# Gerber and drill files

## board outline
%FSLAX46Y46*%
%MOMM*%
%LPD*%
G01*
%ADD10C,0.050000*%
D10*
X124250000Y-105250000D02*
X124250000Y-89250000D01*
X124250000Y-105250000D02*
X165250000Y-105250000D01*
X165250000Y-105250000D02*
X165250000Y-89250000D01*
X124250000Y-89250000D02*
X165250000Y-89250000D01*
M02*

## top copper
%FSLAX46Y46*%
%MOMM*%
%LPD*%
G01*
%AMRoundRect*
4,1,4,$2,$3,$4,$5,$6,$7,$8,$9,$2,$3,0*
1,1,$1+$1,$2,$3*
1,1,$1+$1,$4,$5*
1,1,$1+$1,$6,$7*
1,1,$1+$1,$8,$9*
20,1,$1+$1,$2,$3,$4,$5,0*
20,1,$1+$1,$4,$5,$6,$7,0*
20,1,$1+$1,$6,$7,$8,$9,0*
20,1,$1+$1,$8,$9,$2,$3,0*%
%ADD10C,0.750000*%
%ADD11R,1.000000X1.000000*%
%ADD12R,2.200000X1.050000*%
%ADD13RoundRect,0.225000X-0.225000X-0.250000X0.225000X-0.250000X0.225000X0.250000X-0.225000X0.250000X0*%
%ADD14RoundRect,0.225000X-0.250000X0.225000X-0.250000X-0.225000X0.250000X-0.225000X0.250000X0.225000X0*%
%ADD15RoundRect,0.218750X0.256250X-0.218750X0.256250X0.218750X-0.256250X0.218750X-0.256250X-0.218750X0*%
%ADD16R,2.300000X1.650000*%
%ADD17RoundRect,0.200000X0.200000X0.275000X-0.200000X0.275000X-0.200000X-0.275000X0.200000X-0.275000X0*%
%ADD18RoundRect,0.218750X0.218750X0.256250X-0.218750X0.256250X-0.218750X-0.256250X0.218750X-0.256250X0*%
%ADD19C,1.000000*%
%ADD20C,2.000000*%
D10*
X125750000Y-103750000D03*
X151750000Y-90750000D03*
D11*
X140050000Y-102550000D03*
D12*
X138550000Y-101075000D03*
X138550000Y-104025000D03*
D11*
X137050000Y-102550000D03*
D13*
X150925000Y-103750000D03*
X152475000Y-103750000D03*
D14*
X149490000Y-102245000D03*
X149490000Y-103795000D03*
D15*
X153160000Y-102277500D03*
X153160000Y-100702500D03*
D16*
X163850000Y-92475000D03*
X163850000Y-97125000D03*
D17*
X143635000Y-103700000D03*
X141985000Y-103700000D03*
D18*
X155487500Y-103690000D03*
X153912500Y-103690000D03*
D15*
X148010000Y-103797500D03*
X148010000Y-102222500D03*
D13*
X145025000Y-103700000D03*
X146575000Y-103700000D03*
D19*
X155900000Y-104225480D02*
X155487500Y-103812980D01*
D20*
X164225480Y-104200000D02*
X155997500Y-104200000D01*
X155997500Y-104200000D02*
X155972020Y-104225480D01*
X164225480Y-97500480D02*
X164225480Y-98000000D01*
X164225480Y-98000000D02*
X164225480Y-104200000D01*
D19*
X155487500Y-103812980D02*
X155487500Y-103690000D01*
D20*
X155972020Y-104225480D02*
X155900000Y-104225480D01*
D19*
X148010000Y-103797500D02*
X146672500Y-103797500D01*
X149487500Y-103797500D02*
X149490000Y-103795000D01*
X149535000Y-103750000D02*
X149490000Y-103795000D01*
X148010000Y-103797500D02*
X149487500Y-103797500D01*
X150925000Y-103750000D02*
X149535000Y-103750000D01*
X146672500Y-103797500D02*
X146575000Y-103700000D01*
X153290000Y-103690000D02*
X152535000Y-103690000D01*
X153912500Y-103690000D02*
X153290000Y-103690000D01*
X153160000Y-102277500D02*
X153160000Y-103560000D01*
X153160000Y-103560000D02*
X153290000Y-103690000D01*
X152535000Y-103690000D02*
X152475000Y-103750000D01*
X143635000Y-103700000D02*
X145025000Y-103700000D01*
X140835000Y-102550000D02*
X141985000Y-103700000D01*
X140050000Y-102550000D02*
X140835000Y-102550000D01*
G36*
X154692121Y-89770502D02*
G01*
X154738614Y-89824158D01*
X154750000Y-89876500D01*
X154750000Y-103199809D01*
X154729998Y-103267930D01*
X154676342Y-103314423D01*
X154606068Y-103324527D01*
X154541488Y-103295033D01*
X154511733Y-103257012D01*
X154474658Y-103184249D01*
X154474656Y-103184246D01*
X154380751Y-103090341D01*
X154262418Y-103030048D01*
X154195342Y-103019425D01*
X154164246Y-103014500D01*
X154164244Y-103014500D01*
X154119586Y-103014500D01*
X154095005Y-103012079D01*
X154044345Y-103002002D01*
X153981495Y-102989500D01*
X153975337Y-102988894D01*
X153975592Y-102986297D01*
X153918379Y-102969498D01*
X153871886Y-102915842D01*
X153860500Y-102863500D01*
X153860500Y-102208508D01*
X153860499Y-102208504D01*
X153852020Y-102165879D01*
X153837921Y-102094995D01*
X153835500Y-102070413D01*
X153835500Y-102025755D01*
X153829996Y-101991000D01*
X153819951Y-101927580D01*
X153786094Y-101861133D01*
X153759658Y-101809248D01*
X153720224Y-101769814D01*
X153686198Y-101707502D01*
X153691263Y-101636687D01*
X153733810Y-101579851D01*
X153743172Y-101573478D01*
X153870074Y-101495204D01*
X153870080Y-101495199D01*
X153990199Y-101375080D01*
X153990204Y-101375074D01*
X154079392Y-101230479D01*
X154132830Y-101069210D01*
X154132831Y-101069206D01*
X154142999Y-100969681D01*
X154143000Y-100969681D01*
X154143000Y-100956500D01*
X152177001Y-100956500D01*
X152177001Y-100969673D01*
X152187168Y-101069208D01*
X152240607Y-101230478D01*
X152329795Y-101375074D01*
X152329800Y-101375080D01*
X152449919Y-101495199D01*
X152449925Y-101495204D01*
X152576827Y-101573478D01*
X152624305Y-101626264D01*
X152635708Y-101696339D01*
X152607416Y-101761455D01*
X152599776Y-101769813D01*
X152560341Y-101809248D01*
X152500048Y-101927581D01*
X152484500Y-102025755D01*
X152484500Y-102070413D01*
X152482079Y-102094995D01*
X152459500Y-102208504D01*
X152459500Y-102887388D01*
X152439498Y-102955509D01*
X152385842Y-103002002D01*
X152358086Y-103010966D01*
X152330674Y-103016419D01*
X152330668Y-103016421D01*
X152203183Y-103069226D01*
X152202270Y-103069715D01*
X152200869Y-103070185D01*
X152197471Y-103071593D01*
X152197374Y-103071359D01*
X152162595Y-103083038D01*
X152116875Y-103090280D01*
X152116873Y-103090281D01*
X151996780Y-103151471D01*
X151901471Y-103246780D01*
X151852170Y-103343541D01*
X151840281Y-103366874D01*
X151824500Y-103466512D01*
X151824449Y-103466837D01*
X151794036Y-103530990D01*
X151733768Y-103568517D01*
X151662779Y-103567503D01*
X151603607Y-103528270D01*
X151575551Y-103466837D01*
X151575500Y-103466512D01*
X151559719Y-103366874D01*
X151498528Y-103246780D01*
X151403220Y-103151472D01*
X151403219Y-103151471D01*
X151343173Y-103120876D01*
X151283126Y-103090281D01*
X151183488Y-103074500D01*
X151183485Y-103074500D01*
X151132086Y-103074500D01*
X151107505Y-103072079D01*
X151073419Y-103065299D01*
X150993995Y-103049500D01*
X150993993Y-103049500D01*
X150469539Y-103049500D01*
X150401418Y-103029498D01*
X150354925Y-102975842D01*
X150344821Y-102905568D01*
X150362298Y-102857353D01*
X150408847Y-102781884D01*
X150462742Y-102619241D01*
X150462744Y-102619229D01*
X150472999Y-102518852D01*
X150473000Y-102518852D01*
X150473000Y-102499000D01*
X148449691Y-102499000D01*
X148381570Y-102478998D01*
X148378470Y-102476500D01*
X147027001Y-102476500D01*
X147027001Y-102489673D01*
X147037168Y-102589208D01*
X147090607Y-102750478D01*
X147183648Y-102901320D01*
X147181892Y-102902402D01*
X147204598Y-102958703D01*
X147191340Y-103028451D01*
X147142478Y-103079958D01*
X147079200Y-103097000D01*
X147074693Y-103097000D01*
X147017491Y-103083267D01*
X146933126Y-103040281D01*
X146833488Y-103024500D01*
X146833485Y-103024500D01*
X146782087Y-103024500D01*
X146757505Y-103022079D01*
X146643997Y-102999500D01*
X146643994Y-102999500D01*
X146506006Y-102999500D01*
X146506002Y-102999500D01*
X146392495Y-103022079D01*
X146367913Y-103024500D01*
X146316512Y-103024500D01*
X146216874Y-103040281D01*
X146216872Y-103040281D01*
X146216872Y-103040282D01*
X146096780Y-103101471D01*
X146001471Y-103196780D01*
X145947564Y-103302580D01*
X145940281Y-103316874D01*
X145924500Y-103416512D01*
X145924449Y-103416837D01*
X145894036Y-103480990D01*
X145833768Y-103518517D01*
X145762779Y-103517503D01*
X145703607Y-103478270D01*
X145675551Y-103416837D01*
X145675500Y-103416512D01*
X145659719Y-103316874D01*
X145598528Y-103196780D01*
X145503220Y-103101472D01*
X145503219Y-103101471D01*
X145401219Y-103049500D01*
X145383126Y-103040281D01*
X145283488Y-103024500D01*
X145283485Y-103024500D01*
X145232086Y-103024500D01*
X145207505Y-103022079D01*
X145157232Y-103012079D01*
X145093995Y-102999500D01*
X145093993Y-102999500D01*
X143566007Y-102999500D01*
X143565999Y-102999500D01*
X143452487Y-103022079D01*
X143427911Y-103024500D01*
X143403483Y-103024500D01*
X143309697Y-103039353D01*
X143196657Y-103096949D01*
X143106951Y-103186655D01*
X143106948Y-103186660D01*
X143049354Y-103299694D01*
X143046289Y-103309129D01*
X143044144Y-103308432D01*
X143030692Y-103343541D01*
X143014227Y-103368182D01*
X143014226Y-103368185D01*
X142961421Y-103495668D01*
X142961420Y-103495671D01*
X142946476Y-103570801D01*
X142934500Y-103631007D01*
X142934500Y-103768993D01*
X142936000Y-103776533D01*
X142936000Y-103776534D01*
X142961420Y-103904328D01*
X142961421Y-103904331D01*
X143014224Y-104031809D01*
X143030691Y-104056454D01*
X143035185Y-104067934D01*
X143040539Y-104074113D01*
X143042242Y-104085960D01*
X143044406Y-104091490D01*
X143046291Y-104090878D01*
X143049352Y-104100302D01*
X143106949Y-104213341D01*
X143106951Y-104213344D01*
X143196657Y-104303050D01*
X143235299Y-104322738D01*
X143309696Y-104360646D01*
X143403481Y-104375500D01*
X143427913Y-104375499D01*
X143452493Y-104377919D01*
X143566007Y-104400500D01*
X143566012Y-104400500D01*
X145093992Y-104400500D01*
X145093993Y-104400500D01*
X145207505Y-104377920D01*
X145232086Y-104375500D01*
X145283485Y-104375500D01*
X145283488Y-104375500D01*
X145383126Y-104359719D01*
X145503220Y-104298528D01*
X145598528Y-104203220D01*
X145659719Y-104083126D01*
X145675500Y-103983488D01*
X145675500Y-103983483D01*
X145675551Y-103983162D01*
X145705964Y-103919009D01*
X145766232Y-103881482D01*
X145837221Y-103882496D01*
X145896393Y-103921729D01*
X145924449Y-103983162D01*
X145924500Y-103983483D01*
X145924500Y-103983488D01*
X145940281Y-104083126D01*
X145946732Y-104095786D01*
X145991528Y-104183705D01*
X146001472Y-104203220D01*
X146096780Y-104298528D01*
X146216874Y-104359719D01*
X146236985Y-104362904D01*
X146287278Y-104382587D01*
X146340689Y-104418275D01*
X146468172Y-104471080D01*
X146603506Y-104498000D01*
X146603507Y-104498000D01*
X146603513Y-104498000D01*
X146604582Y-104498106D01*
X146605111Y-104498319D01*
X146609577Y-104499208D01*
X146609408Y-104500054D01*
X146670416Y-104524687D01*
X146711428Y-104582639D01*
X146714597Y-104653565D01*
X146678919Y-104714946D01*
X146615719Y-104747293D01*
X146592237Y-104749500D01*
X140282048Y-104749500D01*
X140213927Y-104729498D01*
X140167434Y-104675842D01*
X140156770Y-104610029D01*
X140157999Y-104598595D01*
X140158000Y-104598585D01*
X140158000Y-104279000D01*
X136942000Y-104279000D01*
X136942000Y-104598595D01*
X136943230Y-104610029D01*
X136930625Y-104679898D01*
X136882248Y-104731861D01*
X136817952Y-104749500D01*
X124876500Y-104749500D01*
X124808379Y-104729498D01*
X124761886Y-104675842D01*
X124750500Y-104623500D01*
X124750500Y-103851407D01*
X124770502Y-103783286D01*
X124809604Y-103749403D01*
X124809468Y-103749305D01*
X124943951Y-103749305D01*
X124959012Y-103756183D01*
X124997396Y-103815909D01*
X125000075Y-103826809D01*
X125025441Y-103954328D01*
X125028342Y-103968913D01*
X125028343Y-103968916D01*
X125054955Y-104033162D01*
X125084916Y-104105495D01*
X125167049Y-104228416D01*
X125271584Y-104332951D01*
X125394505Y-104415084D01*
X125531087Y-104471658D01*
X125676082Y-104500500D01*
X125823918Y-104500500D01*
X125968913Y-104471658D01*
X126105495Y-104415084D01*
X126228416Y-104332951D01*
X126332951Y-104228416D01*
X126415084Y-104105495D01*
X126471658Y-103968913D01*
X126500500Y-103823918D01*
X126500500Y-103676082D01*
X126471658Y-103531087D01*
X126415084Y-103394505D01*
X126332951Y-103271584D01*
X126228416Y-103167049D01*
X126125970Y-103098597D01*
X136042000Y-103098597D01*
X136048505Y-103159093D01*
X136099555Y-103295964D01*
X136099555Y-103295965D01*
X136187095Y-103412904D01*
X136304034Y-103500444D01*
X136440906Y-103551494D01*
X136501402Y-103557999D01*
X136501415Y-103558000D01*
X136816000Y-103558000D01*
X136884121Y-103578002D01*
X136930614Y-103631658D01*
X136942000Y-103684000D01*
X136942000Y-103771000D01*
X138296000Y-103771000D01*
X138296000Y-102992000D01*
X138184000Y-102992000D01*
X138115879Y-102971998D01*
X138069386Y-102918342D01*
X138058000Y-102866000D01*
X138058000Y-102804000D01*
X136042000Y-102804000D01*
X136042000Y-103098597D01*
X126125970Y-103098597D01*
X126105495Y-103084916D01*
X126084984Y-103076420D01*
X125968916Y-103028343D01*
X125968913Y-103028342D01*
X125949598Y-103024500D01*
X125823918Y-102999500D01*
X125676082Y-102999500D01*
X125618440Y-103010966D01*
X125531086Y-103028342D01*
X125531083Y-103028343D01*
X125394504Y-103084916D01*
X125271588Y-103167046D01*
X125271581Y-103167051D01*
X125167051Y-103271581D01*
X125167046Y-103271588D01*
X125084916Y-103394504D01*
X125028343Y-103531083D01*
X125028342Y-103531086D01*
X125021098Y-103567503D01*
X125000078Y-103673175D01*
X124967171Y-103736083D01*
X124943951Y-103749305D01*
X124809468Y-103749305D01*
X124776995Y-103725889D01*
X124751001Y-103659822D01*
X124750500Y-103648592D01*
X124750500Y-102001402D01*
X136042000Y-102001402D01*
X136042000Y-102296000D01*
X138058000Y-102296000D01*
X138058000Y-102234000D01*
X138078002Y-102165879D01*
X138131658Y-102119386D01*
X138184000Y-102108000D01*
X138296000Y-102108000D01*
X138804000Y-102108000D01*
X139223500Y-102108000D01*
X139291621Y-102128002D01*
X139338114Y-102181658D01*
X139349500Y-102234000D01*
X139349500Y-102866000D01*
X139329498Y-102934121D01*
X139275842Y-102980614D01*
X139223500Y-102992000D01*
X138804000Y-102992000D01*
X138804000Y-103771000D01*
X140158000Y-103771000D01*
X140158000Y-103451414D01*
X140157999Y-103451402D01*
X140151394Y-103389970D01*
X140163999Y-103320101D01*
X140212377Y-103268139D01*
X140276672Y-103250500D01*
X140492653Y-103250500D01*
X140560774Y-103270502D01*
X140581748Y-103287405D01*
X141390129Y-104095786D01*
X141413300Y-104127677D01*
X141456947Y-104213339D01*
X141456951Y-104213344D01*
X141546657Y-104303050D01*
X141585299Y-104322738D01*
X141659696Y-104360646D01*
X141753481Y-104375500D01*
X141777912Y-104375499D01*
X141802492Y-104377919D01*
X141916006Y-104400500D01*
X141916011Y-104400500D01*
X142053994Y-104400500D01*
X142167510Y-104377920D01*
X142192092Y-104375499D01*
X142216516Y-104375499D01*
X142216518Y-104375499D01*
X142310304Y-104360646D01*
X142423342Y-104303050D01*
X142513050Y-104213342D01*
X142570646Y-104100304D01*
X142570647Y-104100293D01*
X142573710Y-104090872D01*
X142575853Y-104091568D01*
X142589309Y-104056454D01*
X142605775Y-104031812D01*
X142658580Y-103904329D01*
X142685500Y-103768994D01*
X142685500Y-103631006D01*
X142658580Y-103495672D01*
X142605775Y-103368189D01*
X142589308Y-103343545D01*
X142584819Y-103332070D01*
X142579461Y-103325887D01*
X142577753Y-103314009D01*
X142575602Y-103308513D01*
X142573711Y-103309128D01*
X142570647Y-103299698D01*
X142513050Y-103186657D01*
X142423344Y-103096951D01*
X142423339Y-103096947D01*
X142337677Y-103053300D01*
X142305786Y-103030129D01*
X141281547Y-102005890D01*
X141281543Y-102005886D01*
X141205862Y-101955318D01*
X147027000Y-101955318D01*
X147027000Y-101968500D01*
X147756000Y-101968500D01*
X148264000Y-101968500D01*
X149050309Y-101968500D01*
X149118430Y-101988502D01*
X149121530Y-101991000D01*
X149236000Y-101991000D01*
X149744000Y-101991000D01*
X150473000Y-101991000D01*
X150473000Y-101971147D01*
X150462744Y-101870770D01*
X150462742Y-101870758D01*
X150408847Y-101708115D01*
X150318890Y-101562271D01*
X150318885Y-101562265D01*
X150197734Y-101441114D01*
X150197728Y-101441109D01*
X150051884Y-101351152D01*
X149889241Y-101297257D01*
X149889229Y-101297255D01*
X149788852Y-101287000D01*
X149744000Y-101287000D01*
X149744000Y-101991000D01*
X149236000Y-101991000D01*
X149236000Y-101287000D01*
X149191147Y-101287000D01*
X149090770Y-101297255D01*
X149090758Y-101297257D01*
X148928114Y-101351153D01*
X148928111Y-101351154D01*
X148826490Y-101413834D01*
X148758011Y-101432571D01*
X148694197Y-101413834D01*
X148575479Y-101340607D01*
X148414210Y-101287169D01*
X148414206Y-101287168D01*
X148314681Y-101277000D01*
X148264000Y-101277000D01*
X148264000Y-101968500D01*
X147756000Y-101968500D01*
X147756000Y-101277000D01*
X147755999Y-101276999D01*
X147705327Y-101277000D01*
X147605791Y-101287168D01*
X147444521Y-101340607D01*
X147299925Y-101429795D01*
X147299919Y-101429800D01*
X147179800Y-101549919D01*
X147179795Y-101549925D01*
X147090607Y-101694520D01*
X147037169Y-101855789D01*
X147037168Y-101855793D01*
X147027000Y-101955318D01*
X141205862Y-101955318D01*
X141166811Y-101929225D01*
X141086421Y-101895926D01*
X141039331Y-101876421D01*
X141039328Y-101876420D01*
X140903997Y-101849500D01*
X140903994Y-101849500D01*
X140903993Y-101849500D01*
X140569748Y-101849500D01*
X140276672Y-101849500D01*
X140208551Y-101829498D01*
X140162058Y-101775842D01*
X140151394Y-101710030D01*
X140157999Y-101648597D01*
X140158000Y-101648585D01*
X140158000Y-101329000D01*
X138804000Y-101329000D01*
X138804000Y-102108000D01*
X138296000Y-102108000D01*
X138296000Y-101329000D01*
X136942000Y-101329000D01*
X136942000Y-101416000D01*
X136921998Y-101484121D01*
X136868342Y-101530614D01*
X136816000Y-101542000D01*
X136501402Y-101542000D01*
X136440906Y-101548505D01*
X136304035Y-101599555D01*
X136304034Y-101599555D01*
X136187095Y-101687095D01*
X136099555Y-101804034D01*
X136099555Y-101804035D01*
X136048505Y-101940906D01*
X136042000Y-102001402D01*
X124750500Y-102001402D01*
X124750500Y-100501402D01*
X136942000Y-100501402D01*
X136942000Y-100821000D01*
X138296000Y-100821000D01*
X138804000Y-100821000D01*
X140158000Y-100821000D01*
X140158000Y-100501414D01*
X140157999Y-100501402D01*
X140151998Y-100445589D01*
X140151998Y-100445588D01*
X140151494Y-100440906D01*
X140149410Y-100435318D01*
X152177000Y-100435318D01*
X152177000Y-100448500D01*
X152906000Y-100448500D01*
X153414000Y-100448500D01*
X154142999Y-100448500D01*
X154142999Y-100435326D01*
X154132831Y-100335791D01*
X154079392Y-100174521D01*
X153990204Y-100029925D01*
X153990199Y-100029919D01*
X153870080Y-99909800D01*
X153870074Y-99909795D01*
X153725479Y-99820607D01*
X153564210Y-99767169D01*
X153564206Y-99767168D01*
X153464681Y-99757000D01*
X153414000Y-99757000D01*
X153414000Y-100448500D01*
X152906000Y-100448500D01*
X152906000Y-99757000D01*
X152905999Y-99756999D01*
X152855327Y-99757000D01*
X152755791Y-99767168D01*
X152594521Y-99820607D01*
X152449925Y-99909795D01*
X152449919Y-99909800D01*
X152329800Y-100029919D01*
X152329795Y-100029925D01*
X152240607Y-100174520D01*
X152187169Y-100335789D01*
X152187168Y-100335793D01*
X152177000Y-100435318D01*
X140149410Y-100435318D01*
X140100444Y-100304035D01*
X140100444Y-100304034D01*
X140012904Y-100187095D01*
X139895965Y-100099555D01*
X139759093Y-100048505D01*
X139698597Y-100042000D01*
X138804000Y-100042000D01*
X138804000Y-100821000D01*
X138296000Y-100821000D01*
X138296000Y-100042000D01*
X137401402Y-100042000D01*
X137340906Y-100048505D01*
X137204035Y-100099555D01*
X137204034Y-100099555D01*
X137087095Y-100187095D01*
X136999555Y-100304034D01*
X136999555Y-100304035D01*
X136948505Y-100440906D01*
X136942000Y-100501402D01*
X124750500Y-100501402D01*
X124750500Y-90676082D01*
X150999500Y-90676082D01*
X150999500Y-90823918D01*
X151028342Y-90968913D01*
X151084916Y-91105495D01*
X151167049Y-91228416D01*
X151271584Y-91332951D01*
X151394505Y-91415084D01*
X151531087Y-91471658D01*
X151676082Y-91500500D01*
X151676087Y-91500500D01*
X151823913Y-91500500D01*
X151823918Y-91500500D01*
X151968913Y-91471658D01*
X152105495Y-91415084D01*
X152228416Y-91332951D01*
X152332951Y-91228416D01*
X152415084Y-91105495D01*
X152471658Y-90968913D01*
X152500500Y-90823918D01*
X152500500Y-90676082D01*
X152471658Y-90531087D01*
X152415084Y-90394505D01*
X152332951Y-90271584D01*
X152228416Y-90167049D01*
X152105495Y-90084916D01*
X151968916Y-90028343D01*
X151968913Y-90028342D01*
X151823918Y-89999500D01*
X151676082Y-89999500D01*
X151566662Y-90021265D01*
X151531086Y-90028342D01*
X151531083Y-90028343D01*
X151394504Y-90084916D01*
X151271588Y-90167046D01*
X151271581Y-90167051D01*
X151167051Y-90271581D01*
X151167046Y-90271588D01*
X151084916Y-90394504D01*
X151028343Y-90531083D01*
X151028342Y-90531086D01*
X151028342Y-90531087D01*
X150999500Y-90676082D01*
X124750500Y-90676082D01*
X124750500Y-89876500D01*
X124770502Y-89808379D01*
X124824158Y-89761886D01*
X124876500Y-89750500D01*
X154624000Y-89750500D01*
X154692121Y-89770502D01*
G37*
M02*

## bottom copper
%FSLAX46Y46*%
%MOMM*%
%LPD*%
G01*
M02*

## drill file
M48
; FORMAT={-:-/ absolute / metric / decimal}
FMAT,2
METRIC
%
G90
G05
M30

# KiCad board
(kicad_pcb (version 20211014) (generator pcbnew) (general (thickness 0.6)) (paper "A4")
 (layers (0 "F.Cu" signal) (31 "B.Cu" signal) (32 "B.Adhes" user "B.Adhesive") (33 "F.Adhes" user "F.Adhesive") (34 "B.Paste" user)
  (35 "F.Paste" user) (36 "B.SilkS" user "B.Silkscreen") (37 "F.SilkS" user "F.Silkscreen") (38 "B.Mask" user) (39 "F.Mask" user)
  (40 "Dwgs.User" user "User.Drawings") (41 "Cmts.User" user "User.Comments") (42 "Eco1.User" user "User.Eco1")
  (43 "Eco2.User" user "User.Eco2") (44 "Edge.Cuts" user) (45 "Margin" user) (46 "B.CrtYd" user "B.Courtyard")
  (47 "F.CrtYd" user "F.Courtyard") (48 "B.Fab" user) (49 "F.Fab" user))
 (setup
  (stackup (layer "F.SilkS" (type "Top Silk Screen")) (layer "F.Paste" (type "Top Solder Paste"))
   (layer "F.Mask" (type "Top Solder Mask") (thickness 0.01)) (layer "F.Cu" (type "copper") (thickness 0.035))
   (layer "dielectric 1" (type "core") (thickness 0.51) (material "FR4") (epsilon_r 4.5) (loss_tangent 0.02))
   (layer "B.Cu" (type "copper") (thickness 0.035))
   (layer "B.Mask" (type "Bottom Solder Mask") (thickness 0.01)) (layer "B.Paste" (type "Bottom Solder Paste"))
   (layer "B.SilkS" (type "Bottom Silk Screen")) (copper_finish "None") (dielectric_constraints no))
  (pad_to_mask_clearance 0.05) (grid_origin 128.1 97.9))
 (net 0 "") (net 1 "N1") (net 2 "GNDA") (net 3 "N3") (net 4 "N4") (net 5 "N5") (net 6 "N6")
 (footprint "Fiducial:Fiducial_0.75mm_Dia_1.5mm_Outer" (layer "F.Cu") (at 125.75 103.75)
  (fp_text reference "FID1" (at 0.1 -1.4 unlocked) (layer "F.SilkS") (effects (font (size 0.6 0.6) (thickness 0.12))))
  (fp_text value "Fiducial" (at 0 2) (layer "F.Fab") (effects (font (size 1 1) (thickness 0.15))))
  (pad "" smd circle locked (at 0 0) (size 0.75 0.75) (layers "F.Cu" "F.Mask") (solder_mask_margin 0.375) (clearance 0.375)))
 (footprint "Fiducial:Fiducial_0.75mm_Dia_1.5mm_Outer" (layer "F.Cu") (at 151.75 90.75)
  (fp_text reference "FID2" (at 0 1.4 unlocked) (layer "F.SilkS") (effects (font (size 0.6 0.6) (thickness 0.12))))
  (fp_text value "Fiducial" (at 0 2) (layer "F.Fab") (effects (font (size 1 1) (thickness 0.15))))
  (pad "" smd circle locked (at 0 0) (size 0.75 0.75) (layers "F.Cu" "F.Mask") (solder_mask_margin 0.375) (clearance 0.375)))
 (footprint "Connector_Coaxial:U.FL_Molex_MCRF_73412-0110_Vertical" (layer "F.Cu") (at 138.55 102.55 90)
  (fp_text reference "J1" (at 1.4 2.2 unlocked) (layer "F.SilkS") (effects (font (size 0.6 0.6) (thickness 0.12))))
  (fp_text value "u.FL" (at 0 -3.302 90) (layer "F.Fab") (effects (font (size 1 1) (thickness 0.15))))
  (pad "1" smd rect locked (at 0 1.5 90) (size 1 1) (layers "F.Cu" "F.Paste" "F.Mask") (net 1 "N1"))
  (pad "2" smd rect locked (at 1.475 0 90) (size 1.05 2.2) (layers "F.Cu" "F.Paste" "F.Mask") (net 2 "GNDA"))
  (pad "2" smd rect locked (at -1.475 0 90) (size 1.05 2.2) (layers "F.Cu" "F.Paste" "F.Mask") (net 2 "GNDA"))
  (pad "2" smd rect locked (at 0 -1.5 90) (size 1 1) (layers "F.Cu" "F.Paste" "F.Mask") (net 2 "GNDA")))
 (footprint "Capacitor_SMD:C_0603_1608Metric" (layer "F.Cu") (at 151.7 103.75)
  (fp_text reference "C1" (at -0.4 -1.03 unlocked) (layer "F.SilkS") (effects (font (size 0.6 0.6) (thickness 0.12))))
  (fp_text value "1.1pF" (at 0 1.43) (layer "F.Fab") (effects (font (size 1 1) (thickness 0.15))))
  (pad "1" smd roundrect locked (at -0.775 0) (size 0.9 0.95) (layers "F.Cu" "F.Paste" "F.Mask") (roundrect_rratio 0.25) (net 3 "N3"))
  (pad "2" smd roundrect locked (at 0.775 0) (size 0.9 0.95) (layers "F.Cu" "F.Paste" "F.Mask") (roundrect_rratio 0.25) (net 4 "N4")))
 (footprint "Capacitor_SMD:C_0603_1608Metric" (layer "F.Cu") (at 149.49 103.02 -90)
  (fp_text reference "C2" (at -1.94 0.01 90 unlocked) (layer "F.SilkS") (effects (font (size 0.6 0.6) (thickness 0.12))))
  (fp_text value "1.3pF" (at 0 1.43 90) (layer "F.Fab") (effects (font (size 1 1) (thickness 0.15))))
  (pad "1" smd roundrect locked (at -0.775 0 270) (size 0.9 0.95) (layers "F.Cu" "F.Paste" "F.Mask") (roundrect_rratio 0.25) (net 2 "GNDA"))
  (pad "2" smd roundrect locked (at 0.775 0 270) (size 0.9 0.95) (layers "F.Cu" "F.Paste" "F.Mask") (roundrect_rratio 0.25) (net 3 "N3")))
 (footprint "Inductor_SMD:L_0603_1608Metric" (layer "F.Cu") (at 153.16 101.49 90)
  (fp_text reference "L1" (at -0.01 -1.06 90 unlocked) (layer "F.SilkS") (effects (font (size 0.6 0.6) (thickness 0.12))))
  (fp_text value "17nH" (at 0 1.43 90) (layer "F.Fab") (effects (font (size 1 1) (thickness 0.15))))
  (pad "1" smd roundrect locked (at -0.7875 0 90) (size 0.875 0.95) (layers "F.Cu" "F.Paste" "F.Mask") (roundrect_rratio 0.25) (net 4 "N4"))
  (pad "2" smd roundrect locked (at 0.7875 0 90) (size 0.875 0.95) (layers "F.Cu" "F.Paste" "F.Mask") (roundrect_rratio 0.25) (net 2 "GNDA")))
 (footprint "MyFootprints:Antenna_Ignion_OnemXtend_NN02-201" (layer "F.Cu") (at 163.85 94.8 -90)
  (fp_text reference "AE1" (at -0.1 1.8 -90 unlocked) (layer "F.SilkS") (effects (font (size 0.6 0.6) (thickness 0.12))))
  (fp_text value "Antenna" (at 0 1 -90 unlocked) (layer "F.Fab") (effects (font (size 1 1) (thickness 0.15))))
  (pad "" smd rect (at -2.325 0 270) (size 1.65 2.3) (layers "F.Cu" "F.Paste" "F.Mask"))
  (pad "1" smd rect (at 2.325 0 270) (size 1.65 2.3) (layers "F.Cu" "F.Paste" "F.Mask") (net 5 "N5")))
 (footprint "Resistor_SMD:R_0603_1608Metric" (layer "F.Cu") (at 142.81 103.7 180)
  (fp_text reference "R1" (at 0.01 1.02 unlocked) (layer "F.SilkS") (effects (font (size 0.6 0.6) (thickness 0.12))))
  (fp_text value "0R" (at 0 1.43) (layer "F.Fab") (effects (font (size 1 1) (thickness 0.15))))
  (pad "1" smd roundrect locked (at -0.825 0 180) (size 0.8 0.95) (layers "F.Cu" "F.Paste" "F.Mask") (roundrect_rratio 0.25) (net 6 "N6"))
  (pad "2" smd roundrect locked (at 0.825 0 180) (size 0.8 0.95) (layers "F.Cu" "F.Paste" "F.Mask") (roundrect_rratio 0.25) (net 1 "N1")))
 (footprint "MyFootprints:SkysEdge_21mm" (layer "F.Cu") (at 133.3 91.8)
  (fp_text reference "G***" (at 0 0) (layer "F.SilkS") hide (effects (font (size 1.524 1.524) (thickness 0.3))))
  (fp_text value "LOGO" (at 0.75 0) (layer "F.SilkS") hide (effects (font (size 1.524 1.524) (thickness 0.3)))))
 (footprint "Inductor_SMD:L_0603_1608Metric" (layer "F.Cu") (at 154.7 103.69 180)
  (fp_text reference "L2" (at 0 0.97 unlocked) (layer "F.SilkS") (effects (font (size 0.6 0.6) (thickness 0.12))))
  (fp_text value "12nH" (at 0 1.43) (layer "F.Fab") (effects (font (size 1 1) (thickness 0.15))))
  (pad "1" smd roundrect locked (at -0.7875 0 180) (size 0.875 0.95) (layers "F.Cu" "F.Paste" "F.Mask") (roundrect_rratio 0.25) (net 5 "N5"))
  (pad "2" smd roundrect locked (at 0.7875 0 180) (size 0.875 0.95) (layers "F.Cu" "F.Paste" "F.Mask") (roundrect_rratio 0.25) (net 4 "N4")))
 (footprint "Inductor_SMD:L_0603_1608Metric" (layer "F.Cu") (at 148.01 103.01 90)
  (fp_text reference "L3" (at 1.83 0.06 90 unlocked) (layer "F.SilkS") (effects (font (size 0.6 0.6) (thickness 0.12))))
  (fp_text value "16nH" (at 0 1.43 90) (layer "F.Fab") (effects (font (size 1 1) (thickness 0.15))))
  (pad "1" smd roundrect locked (at -0.7875 0 90) (size 0.875 0.95) (layers "F.Cu" "F.Paste" "F.Mask") (roundrect_rratio 0.25) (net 3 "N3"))
  (pad "2" smd roundrect locked (at 0.7875 0 90) (size 0.875 0.95) (layers "F.Cu" "F.Paste" "F.Mask") (roundrect_rratio 0.25) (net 2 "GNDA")))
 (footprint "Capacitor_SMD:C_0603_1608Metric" (layer "F.Cu") (at 145.8 103.7)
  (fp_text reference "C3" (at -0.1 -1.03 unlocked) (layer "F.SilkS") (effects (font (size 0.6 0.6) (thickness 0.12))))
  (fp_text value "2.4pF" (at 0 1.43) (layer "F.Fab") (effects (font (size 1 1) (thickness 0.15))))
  (pad "1" smd roundrect locked (at -0.775 0) (size 0.9 0.95) (layers "F.Cu" "F.Paste" "F.Mask") (roundrect_rratio 0.25) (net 6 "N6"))
  (pad "2" smd roundrect locked (at 0.775 0) (size 0.9 0.95) (layers "F.Cu" "F.Paste" "F.Mask") (roundrect_rratio 0.25) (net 3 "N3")))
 (gr_line (start 124.25 105.25) (end 124.25 89.25) (layer "Edge.Cuts") (width 0.05))
 (gr_line (start 124.25 105.25) (end 165.25 105.25) (layer "Edge.Cuts") (width 0.05))
 (gr_line (start 165.25 105.25) (end 165.25 89.25) (layer "Edge.Cuts") (width 0.05))
 (gr_line (start 124.25 89.25) (end 165.25 89.25) (layer "Edge.Cuts") (width 0.05))
 (segment (start 155.9 104.22548) (end 155.4875 103.81298) (width 1) (layer "F.Cu") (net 5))
 (segment (start 164.22548 104.2) (end 155.9975 104.2) (width 2) (layer "F.Cu") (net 5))
 (segment (start 155.9975 104.2) (end 155.97202 104.22548) (width 2) (layer "F.Cu") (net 5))
 (segment (start 164.22548 97.50048) (end 164.22548 98) (width 2) (layer "F.Cu") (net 5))
 (segment (start 164.22548 98) (end 164.22548 104.2) (width 2) (layer "F.Cu") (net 5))
 (segment (start 155.4875 103.81298) (end 155.4875 103.69) (width 1) (layer "F.Cu") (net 5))
 (segment (start 155.97202 104.22548) (end 155.9 104.22548) (width 2) (layer "F.Cu") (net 5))
 (segment (start 148.01 103.7975) (end 146.6725 103.7975) (width 1) (layer "F.Cu") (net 3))
 (segment (start 149.4875 103.7975) (end 149.49 103.795) (width 1) (layer "F.Cu") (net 3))
 (segment (start 149.535 103.75) (end 149.49 103.795) (width 1) (layer "F.Cu") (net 3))
 (segment (start 148.01 103.7975) (end 149.4875 103.7975) (width 1) (layer "F.Cu") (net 3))
 (segment (start 150.925 103.75) (end 149.535 103.75) (width 1) (layer "F.Cu") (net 3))
 (segment (start 146.6725 103.7975) (end 146.575 103.7) (width 1) (layer "F.Cu") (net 3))
 (segment (start 153.29 103.69) (end 152.535 103.69) (width 1) (layer "F.Cu") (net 4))
 (segment (start 153.9125 103.69) (end 153.29 103.69) (width 1) (layer "F.Cu") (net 4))
 (segment (start 153.16 102.2775) (end 153.16 103.56) (width 1) (layer "F.Cu") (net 4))
 (segment (start 153.16 103.56) (end 153.29 103.69) (width 1) (layer "F.Cu") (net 4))
 (segment (start 152.535 103.69) (end 152.475 103.75) (width 1) (layer "F.Cu") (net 4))
 (segment (start 143.635 103.7) (end 145.025 103.7) (width 1) (layer "F.Cu") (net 6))
 (segment (start 140.835 102.55) (end 141.985 103.7) (width 1) (layer "F.Cu") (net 1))
 (segment (start 140.05 102.55) (end 140.835 102.55) (width 1) (layer "F.Cu") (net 1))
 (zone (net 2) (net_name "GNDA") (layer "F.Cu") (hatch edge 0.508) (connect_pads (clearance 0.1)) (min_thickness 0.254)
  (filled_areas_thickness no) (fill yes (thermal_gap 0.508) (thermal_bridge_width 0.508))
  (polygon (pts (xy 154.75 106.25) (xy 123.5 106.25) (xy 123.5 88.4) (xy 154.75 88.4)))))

